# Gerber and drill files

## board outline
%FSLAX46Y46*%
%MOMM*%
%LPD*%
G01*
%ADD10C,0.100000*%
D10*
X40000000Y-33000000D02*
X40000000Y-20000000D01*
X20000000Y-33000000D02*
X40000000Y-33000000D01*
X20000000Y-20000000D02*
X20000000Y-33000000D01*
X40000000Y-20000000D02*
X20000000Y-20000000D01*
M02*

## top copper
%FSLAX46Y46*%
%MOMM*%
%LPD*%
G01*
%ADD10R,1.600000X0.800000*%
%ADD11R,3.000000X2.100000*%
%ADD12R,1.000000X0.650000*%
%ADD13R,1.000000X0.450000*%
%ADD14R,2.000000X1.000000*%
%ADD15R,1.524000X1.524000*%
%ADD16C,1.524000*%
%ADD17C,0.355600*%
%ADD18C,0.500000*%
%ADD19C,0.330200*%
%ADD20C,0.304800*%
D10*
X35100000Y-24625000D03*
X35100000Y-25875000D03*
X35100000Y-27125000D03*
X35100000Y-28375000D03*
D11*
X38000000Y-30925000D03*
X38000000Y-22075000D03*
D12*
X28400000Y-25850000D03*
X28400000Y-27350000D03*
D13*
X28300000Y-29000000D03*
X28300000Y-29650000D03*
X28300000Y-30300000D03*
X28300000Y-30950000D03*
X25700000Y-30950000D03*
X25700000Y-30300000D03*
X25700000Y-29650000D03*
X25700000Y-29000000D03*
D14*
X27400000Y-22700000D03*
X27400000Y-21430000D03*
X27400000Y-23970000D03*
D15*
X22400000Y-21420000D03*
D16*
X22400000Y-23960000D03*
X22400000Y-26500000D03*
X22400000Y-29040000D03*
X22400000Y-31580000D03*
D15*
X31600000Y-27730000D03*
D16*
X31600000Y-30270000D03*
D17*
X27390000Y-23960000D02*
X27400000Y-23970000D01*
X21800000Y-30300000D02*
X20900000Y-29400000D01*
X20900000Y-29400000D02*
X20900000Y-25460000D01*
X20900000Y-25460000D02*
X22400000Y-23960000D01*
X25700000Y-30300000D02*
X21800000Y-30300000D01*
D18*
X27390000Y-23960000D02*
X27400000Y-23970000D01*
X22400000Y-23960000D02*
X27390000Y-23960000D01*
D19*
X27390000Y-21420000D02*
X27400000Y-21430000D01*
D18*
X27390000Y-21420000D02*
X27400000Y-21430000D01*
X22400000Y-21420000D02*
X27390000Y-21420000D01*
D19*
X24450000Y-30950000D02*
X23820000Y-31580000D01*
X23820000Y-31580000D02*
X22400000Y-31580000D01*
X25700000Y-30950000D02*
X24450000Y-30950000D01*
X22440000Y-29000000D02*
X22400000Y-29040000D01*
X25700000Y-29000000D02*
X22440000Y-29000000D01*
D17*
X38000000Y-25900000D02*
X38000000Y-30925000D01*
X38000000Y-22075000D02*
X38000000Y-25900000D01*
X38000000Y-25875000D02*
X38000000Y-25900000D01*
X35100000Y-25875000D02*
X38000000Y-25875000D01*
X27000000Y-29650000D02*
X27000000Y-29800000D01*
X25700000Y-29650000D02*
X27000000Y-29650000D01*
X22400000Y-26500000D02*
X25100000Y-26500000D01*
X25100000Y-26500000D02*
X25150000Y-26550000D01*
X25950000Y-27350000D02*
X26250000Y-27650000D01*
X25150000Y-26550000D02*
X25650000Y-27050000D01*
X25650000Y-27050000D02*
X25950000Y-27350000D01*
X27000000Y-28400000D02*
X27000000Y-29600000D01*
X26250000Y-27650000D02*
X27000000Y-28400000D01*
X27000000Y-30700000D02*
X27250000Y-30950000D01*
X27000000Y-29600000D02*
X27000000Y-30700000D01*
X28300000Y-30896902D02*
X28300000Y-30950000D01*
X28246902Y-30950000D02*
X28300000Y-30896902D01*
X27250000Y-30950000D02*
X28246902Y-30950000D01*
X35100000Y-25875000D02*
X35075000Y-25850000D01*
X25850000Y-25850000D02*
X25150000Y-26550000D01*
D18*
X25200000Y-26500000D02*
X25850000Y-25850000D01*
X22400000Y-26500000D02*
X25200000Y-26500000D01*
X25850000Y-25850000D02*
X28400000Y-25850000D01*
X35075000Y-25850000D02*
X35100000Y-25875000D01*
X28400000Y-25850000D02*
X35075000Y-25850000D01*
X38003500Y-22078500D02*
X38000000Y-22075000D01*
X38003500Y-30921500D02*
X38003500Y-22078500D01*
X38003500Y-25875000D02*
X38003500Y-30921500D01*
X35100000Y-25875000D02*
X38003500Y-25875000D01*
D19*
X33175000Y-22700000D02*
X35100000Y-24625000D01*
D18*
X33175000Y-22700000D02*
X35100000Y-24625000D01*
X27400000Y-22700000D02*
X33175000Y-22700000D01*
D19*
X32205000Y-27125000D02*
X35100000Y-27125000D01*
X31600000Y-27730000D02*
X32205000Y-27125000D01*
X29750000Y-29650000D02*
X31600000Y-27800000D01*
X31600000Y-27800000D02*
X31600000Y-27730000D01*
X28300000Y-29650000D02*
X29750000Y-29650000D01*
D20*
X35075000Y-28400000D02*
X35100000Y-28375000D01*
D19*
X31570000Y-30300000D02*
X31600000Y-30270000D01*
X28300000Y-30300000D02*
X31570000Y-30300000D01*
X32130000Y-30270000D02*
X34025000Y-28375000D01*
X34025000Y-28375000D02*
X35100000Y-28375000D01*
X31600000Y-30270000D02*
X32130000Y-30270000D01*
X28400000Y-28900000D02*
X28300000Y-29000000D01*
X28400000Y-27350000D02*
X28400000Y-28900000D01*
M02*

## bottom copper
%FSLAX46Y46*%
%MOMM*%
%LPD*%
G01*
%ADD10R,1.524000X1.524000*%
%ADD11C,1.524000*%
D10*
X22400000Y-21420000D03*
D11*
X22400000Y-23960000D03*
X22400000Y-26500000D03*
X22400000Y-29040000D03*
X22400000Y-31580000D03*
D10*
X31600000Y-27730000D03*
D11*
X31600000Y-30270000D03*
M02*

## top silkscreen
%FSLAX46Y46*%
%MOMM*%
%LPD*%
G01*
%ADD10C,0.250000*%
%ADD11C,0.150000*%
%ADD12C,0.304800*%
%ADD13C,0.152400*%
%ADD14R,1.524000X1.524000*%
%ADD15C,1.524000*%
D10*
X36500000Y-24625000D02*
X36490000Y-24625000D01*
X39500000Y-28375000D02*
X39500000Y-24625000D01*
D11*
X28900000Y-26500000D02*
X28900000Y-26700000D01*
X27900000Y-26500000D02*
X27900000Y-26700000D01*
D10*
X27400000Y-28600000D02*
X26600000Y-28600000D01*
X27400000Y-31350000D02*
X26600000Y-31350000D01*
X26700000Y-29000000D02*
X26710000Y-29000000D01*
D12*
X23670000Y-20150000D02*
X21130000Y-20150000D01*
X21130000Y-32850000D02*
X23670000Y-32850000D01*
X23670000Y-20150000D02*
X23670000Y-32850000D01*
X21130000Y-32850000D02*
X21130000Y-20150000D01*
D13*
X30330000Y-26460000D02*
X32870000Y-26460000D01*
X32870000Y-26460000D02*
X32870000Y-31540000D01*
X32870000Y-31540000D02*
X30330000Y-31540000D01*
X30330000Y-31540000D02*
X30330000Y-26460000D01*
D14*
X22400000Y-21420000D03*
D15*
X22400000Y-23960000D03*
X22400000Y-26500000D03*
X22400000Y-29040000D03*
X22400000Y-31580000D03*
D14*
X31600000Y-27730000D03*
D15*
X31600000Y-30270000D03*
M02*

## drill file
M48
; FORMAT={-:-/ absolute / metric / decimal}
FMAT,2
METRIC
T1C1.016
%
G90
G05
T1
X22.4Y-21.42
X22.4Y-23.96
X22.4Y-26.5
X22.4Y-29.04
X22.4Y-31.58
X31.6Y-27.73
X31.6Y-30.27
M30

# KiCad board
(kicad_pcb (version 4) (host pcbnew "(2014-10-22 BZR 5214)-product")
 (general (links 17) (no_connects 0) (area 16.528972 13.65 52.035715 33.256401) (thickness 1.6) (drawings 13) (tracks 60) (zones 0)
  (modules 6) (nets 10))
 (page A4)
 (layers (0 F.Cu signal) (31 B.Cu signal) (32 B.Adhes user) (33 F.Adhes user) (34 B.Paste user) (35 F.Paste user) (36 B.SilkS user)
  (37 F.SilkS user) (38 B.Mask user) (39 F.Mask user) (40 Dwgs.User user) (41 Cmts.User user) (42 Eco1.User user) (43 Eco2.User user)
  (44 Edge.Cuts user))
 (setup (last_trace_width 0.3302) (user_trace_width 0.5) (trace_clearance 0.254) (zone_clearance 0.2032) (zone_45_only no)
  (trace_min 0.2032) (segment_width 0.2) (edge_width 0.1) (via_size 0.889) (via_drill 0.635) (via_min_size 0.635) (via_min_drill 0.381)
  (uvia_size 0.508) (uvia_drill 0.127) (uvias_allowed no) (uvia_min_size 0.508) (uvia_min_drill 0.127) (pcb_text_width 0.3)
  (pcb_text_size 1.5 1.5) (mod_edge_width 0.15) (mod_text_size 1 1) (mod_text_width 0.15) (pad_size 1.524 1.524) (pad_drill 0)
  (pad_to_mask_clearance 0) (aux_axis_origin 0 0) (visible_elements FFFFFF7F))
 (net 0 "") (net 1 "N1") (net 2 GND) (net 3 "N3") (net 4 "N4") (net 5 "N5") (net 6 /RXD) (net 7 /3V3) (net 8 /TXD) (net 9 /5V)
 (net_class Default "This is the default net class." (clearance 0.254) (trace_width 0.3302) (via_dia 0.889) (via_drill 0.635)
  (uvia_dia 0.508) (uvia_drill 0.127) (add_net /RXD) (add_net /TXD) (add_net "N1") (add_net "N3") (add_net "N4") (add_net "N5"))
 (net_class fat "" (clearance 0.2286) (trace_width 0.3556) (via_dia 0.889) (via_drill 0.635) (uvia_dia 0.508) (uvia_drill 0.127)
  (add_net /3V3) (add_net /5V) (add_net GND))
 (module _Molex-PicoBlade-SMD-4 (layer F.Cu) (at 38 26.5 90)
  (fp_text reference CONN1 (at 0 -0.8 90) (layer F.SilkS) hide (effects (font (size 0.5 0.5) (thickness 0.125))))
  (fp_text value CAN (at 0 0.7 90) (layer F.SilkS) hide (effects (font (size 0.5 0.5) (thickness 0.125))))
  (fp_line (start 1.875 -1.5) (end 1.875 -1.51) (layer F.SilkS) (width 0.25))
  (fp_line (start -1.875 1.5) (end 1.875 1.5) (layer F.SilkS) (width 0.25))
  (pad 1 smd rect (at 1.875 -2.9 90) (size 0.8 1.6) (layers F.Cu F.Paste F.Mask) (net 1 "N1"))
  (pad 2 smd rect (at 0.625 -2.9 90) (size 0.8 1.6) (layers F.Cu F.Paste F.Mask) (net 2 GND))
  (pad 3 smd rect (at -0.625 -2.9 90) (size 0.8 1.6) (layers F.Cu F.Paste F.Mask) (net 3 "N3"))
  (pad 4 smd rect (at -1.875 -2.9 90) (size 0.8 1.6) (layers F.Cu F.Paste F.Mask) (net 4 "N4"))
  (pad MECH smd rect (at -4.425 0 90) (size 2.1 3) (layers F.Cu F.Paste F.Mask) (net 2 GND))
  (pad MECH smd rect (at 4.425 0 90) (size 2.1 3) (layers F.Cu F.Paste F.Mask) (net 2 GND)))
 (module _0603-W (layer F.Cu) (at 28.4 26.6 90)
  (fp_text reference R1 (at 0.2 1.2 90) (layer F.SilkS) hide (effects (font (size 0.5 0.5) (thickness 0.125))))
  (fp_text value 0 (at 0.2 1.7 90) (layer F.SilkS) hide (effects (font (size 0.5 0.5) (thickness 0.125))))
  (fp_line (start 0.1 0.5) (end -0.1 0.5) (layer F.SilkS) (width 0.15))
  (fp_line (start 0.1 -0.5) (end -0.1 -0.5) (layer F.SilkS) (width 0.15))
  (pad 2 smd rect (at 0.75 0 90) (size 0.65 1) (layers F.Cu F.Paste F.Mask) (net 2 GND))
  (pad 1 smd rect (at -0.75 0 90) (size 0.65 1) (layers F.Cu F.Paste F.Mask) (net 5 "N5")))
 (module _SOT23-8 (layer F.Cu) (at 25.7 29 270) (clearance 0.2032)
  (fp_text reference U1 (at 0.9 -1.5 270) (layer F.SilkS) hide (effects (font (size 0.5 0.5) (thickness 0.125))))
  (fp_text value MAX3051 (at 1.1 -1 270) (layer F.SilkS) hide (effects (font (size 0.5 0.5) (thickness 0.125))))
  (fp_line (start -0.4 -1.7) (end -0.4 -0.9) (layer F.SilkS) (width 0.25))
  (fp_line (start 2.35 -1.7) (end 2.35 -0.9) (layer F.SilkS) (width 0.25))
  (fp_line (start 0 -1) (end 0 -1.01) (layer F.SilkS) (width 0.25))
  (pad 8 smd rect (at 0 -2.6 270) (size 0.45 1) (layers F.Cu F.Paste F.Mask) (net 5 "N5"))
  (pad 7 smd rect (at 0.65 -2.6 270) (size 0.45 1) (layers F.Cu F.Paste F.Mask) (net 3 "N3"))
  (pad 6 smd rect (at 1.3 -2.6 270) (size 0.45 1) (layers F.Cu F.Paste F.Mask) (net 4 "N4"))
  (pad 5 smd rect (at 1.95 -2.6 270) (size 0.45 1) (layers F.Cu F.Paste F.Mask) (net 2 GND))
  (pad 4 smd rect (at 1.95 0 270) (size 0.45 1) (layers F.Cu F.Paste F.Mask) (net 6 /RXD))
  (pad 3 smd rect (at 1.3 0 270) (size 0.45 1) (layers F.Cu F.Paste F.Mask) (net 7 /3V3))
  (pad 2 smd rect (at 0.65 0 270) (size 0.45 1) (layers F.Cu F.Paste F.Mask) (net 2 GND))
  (pad 1 smd rect (at 0 0 270) (size 0.45 1) (layers F.Cu F.Paste F.Mask) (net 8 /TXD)))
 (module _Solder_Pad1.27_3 (layer F.Cu) (at 27.4 22.7 270)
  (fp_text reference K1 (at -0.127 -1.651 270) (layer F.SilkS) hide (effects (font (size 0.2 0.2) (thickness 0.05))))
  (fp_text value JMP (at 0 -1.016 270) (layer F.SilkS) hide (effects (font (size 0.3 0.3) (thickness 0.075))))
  (pad 2 smd rect (at 0 0 270) (size 1 2) (layers F.Cu F.Paste F.Mask) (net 1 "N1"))
  (pad 1 smd rect (at -1.27 0 270) (size 1 2) (layers F.Cu F.Paste F.Mask) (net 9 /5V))
  (pad 3 smd rect (at 1.27 0 270) (size 1 2) (layers F.Cu F.Paste F.Mask) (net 7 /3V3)))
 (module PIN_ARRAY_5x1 (layer F.Cu) (at 22.4 26.5 270)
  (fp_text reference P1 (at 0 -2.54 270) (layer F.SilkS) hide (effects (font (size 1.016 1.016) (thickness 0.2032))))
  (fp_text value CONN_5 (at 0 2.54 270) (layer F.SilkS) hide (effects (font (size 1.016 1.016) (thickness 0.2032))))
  (fp_line (start -6.35 -1.27) (end -6.35 1.27) (layer F.SilkS) (width 0.3048))
  (fp_line (start 6.35 1.27) (end 6.35 -1.27) (layer F.SilkS) (width 0.3048))
  (fp_line (start -6.35 -1.27) (end 6.35 -1.27) (layer F.SilkS) (width 0.3048))
  (fp_line (start 6.35 1.27) (end -6.35 1.27) (layer F.SilkS) (width 0.3048))
  (pad 1 thru_hole rect (at -5.08 0 270) (size 1.524 1.524) (drill 1.016) (layers *.Cu *.Mask F.SilkS) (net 9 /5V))
  (pad 2 thru_hole circle (at -2.54 0 270) (size 1.524 1.524) (drill 1.016) (layers *.Cu *.Mask F.SilkS) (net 7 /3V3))
  (pad 3 thru_hole circle (at 0 0 270) (size 1.524 1.524) (drill 1.016) (layers *.Cu *.Mask F.SilkS) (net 2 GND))
  (pad 4 thru_hole circle (at 2.54 0 270) (size 1.524 1.524) (drill 1.016) (layers *.Cu *.Mask F.SilkS) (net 8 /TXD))
  (pad 5 thru_hole circle (at 5.08 0 270) (size 1.524 1.524) (drill 1.016) (layers *.Cu *.Mask F.SilkS) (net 6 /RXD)))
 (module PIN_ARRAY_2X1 (layer F.Cu) (at 31.6 29 270)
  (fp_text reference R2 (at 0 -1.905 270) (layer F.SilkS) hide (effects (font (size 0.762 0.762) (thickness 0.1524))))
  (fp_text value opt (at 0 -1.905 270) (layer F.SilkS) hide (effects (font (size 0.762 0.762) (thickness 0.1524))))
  (fp_line (start -2.54 1.27) (end -2.54 -1.27) (layer F.SilkS) (width 0.1524))
  (fp_line (start -2.54 -1.27) (end 2.54 -1.27) (layer F.SilkS) (width 0.1524))
  (fp_line (start 2.54 -1.27) (end 2.54 1.27) (layer F.SilkS) (width 0.1524))
  (fp_line (start 2.54 1.27) (end -2.54 1.27) (layer F.SilkS) (width 0.1524))
  (pad 1 thru_hole rect (at -1.27 0 270) (size 1.524 1.524) (drill 1.016) (layers *.Cu *.Mask F.SilkS) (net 3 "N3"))
  (pad 2 thru_hole circle (at 1.27 0 270) (size 1.524 1.524) (drill 1.016) (layers *.Cu *.Mask F.SilkS) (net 4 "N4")))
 (gr_line (start 40 33) (end 40 20) (angle 90) (layer Edge.Cuts) (width 0.1))
 (gr_line (start 20 33) (end 40 33) (angle 90) (layer Edge.Cuts) (width 0.1))
 (gr_line (start 20 20) (end 20 33) (angle 90) (layer Edge.Cuts) (width 0.1))
 (gr_line (start 40 20) (end 20 20) (angle 90) (layer Edge.Cuts) (width 0.1))
 (segment (start 27.39 23.96) (end 27.4 23.97) (width 0.3556) (layer F.Cu) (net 7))
 (segment (start 21.8 30.3) (end 20.9 29.4) (width 0.3556) (layer F.Cu) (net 7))
 (segment (start 20.9 29.4) (end 20.9 25.46) (width 0.3556) (layer F.Cu) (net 7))
 (segment (start 20.9 25.46) (end 22.4 23.96) (width 0.3556) (layer F.Cu) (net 7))
 (segment (start 25.7 30.3) (end 21.8 30.3) (width 0.3556) (layer F.Cu) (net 7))
 (segment (start 27.39 23.96) (end 27.4 23.97) (width 0.5) (layer F.Cu) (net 7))
 (segment (start 22.4 23.96) (end 27.39 23.96) (width 0.5) (layer F.Cu) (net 7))
 (segment (start 27.39 21.42) (end 27.4 21.43) (width 0.3302) (layer F.Cu) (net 9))
 (segment (start 27.39 21.42) (end 27.4 21.43) (width 0.5) (layer F.Cu) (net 9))
 (segment (start 22.4 21.42) (end 27.39 21.42) (width 0.5) (layer F.Cu) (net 9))
 (segment (start 24.45 30.95) (end 23.82 31.58) (width 0.3302) (layer F.Cu) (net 6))
 (segment (start 23.82 31.58) (end 22.4 31.58) (width 0.3302) (layer F.Cu) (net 6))
 (segment (start 25.7 30.95) (end 24.45 30.95) (width 0.3302) (layer F.Cu) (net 6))
 (segment (start 22.44 29) (end 22.4 29.04) (width 0.3302) (layer F.Cu) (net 8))
 (segment (start 25.7 29) (end 22.44 29) (width 0.3302) (layer F.Cu) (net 8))
 (segment (start 38 25.9) (end 38 30.925) (width 0.3556) (layer F.Cu) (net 2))
 (segment (start 38 22.075) (end 38 25.9) (width 0.3556) (layer F.Cu) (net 2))
 (segment (start 38 25.875) (end 38 25.9) (width 0.3556) (layer F.Cu) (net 2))
 (segment (start 35.1 25.875) (end 38 25.875) (width 0.3556) (layer F.Cu) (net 2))
 (segment (start 27 29.65) (end 27 29.8) (width 0.3556) (layer F.Cu) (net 2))
 (segment (start 25.7 29.65) (end 27 29.65) (width 0.3556) (layer F.Cu) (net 2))
 (segment (start 22.4 26.5) (end 25.1 26.5) (width 0.3556) (layer F.Cu) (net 2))
 (segment (start 25.1 26.5) (end 25.15 26.55) (width 0.3556) (layer F.Cu) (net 2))
 (segment (start 25.95 27.35) (end 26.25 27.65) (width 0.3556) (layer F.Cu) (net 2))
 (segment (start 25.15 26.55) (end 25.65 27.05) (width 0.3556) (layer F.Cu) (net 2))
 (segment (start 25.65 27.05) (end 25.95 27.35) (width 0.3556) (layer F.Cu) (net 2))
 (segment (start 27 28.4) (end 27 29.6) (width 0.3556) (layer F.Cu) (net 2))
 (segment (start 26.25 27.65) (end 27 28.4) (width 0.3556) (layer F.Cu) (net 2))
 (segment (start 27 30.7) (end 27.25 30.95) (width 0.3556) (layer F.Cu) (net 2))
 (segment (start 27 29.6) (end 27 30.7) (width 0.3556) (layer F.Cu) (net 2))
 (segment (start 28.3 30.896902) (end 28.3 30.95) (width 0.3556) (layer F.Cu) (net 2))
 (segment (start 28.246902 30.95) (end 28.3 30.896902) (width 0.3556) (layer F.Cu) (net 2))
 (segment (start 27.25 30.95) (end 28.246902 30.95) (width 0.3556) (layer F.Cu) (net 2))
 (segment (start 35.1 25.875) (end 35.075 25.85) (width 0.3556) (layer F.Cu) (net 2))
 (segment (start 25.85 25.85) (end 25.15 26.55) (width 0.3556) (layer F.Cu) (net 2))
 (segment (start 25.2 26.5) (end 25.85 25.85) (width 0.5) (layer F.Cu) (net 2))
 (segment (start 22.4 26.5) (end 25.2 26.5) (width 0.5) (layer F.Cu) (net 2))
 (segment (start 25.85 25.85) (end 28.4 25.85) (width 0.5) (layer F.Cu) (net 2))
 (segment (start 35.075 25.85) (end 35.1 25.875) (width 0.5) (layer F.Cu) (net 2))
 (segment (start 28.4 25.85) (end 35.075 25.85) (width 0.5) (layer F.Cu) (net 2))
 (segment (start 38.0035 22.0785) (end 38 22.075) (width 0.5) (layer F.Cu) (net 2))
 (segment (start 38.0035 30.9215) (end 38.0035 22.0785) (width 0.5) (layer F.Cu) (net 2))
 (segment (start 38.0035 25.875) (end 38.0035 30.9215) (width 0.5) (layer F.Cu) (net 2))
 (segment (start 35.1 25.875) (end 38.0035 25.875) (width 0.5) (layer F.Cu) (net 2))
 (segment (start 33.175 22.7) (end 35.1 24.625) (width 0.3302) (layer F.Cu) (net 1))
 (segment (start 33.175 22.7) (end 35.1 24.625) (width 0.5) (layer F.Cu) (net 1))
 (segment (start 27.4 22.7) (end 33.175 22.7) (width 0.5) (layer F.Cu) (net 1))
 (segment (start 32.205 27.125) (end 35.1 27.125) (width 0.3302) (layer F.Cu) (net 3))
 (segment (start 31.6 27.73) (end 32.205 27.125) (width 0.3302) (layer F.Cu) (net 3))
 (segment (start 29.75 29.65) (end 31.6 27.8) (width 0.3302) (layer F.Cu) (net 3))
 (segment (start 31.6 27.8) (end 31.6 27.73) (width 0.3302) (layer F.Cu) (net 3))
 (segment (start 28.3 29.65) (end 29.75 29.65) (width 0.3302) (layer F.Cu) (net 3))
 (segment (start 35.075 28.4) (end 35.1 28.375) (width 0.3048) (layer F.Cu) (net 4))
 (segment (start 31.57 30.3) (end 31.6 30.27) (width 0.3302) (layer F.Cu) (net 4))
 (segment (start 28.3 30.3) (end 31.57 30.3) (width 0.3302) (layer F.Cu) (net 4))
 (segment (start 32.13 30.27) (end 34.025 28.375) (width 0.3302) (layer F.Cu) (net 4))
 (segment (start 34.025 28.375) (end 35.1 28.375) (width 0.3302) (layer F.Cu) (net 4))
 (segment (start 31.6 30.27) (end 32.13 30.27) (width 0.3302) (layer F.Cu) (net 4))
 (segment (start 28.4 28.9) (end 28.3 29) (width 0.3302) (layer F.Cu) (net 5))
 (segment (start 28.4 27.35) (end 28.4 28.9) (width 0.3302) (layer F.Cu) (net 5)))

